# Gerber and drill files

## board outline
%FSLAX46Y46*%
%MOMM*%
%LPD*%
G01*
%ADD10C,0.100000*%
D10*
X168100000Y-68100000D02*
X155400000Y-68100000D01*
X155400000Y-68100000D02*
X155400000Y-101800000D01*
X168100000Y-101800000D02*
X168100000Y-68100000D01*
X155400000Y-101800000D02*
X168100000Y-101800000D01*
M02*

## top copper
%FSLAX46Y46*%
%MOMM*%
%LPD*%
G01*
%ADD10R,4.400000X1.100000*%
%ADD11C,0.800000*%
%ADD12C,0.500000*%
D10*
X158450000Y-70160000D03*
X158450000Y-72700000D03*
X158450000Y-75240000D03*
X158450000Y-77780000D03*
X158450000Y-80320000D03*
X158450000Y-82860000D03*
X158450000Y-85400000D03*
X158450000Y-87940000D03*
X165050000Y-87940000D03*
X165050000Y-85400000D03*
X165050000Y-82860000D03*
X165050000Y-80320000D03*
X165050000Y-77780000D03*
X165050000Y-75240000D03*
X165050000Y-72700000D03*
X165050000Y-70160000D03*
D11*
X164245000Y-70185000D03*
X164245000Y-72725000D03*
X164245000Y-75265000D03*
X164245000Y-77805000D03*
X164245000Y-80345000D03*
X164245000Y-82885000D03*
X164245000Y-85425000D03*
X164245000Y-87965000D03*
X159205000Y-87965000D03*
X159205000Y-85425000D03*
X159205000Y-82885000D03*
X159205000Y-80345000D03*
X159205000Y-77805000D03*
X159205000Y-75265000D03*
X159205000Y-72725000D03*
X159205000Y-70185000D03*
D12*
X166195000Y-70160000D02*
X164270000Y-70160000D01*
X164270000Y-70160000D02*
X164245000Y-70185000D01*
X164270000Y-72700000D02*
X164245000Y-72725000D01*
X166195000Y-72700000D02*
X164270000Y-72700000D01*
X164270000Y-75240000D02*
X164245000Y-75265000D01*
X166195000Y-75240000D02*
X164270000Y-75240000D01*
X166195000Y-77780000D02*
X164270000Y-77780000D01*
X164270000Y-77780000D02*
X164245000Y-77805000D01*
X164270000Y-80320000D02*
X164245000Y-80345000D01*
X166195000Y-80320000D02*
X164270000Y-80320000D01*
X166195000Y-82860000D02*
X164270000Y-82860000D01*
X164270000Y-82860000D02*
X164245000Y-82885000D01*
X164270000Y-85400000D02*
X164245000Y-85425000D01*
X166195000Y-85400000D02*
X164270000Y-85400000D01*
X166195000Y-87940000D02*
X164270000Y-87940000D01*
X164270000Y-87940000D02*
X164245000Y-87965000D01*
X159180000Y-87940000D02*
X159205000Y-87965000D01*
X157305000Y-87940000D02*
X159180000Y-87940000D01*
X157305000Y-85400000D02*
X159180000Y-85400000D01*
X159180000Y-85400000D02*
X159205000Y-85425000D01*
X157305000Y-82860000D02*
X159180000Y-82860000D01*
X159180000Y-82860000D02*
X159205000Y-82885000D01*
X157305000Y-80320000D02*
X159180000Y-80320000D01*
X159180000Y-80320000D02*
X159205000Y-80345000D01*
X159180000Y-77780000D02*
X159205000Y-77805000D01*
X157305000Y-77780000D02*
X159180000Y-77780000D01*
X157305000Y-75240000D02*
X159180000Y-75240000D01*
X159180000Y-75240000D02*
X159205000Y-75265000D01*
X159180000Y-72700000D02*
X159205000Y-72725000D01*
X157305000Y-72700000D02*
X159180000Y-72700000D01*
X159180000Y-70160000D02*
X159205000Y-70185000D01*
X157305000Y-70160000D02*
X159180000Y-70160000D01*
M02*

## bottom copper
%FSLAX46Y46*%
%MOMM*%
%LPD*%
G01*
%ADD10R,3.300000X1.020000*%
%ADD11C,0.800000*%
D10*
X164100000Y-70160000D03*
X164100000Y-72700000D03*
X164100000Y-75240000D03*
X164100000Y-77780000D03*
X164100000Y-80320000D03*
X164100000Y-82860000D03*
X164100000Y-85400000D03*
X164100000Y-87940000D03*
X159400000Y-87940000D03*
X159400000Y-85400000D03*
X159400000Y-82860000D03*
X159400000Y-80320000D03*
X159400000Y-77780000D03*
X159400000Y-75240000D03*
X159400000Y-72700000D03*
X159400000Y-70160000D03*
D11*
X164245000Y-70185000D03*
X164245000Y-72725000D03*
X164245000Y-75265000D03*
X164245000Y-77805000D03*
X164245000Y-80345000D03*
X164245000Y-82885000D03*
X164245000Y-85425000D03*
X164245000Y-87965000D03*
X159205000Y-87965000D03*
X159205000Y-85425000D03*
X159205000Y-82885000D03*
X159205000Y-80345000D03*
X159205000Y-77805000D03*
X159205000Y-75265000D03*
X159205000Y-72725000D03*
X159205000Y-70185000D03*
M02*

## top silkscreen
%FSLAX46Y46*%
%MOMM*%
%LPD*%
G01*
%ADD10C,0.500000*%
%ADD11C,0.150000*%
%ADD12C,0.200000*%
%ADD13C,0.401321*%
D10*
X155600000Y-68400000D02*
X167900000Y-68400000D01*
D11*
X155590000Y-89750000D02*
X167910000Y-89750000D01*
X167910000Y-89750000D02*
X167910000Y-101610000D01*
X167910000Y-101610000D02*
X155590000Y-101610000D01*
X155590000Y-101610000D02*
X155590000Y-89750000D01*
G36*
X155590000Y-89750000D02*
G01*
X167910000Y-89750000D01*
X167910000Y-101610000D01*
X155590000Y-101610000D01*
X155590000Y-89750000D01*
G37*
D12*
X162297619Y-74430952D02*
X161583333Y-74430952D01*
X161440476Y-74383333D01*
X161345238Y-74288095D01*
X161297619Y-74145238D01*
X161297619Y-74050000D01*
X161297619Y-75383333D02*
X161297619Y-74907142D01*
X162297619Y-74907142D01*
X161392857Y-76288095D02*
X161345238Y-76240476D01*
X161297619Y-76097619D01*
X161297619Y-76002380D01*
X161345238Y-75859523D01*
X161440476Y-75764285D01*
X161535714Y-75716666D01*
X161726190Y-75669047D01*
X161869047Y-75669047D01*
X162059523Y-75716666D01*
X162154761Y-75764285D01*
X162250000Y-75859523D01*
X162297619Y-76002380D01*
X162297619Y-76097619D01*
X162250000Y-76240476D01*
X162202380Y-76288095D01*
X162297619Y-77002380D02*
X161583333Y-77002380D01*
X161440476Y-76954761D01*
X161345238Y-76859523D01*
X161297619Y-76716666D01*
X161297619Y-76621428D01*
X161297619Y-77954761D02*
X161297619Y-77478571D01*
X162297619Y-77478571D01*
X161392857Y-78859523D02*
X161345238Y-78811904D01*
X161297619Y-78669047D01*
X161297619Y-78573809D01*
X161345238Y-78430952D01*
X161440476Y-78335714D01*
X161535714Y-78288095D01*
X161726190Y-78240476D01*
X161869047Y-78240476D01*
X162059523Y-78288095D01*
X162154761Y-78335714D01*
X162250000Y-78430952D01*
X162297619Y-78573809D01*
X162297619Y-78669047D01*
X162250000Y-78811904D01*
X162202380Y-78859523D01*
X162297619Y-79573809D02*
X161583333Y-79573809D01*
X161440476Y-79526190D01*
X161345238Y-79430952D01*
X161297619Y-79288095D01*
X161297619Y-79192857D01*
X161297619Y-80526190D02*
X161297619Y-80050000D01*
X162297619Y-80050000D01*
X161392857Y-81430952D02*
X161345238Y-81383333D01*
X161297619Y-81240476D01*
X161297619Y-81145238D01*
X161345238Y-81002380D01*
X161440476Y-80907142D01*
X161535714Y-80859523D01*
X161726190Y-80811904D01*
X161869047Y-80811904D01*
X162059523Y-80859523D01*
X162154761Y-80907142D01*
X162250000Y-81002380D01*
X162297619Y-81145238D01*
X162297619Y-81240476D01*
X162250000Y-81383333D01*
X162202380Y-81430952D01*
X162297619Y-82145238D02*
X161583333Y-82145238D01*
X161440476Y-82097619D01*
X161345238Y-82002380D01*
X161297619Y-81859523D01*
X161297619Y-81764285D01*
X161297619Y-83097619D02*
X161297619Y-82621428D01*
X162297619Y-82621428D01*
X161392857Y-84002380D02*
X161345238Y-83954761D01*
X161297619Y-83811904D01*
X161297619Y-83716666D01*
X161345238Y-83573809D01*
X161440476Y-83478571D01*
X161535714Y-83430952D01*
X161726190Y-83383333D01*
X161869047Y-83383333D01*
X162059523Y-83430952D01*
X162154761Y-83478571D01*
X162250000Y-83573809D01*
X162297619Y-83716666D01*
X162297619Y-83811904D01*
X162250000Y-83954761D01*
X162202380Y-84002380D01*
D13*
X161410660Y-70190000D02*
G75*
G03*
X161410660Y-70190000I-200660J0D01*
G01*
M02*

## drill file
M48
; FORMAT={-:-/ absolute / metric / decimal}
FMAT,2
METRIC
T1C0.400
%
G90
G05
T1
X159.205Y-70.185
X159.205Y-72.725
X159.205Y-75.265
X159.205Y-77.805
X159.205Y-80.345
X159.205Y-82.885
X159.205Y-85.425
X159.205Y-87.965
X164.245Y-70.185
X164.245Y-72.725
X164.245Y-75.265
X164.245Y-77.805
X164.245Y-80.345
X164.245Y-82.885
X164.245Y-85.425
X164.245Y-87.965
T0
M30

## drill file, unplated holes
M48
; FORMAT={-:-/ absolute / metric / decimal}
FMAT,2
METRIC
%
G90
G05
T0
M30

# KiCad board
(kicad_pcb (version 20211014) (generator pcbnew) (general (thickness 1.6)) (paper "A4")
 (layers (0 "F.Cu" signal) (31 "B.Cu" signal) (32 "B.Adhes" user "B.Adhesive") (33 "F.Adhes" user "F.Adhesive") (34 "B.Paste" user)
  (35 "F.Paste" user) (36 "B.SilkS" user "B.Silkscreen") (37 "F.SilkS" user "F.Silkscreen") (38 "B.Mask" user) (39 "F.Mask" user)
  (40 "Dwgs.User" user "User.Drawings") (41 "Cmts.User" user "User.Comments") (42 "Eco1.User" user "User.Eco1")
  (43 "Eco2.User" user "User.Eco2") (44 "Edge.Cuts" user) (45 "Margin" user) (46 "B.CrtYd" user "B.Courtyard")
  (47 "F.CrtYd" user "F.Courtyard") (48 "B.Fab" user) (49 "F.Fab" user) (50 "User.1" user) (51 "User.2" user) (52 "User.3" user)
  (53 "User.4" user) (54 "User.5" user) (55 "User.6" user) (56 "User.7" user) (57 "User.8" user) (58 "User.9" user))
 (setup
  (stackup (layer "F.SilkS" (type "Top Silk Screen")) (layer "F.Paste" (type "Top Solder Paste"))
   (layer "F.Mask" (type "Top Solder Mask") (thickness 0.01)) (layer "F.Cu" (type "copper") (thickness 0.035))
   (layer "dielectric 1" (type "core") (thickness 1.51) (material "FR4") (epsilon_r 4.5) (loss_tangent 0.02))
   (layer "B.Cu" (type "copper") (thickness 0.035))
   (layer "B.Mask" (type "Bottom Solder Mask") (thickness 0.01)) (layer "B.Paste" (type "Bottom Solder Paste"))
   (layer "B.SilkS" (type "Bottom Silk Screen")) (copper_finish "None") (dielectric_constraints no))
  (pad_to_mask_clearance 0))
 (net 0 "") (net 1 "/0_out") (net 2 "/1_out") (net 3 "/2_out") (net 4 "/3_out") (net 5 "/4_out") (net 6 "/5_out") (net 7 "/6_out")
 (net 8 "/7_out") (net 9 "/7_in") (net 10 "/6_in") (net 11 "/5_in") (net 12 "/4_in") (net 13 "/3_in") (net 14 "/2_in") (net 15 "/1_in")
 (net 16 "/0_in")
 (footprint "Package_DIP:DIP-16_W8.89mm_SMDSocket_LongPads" (layer "F.Cu") (at 161.75 79.05)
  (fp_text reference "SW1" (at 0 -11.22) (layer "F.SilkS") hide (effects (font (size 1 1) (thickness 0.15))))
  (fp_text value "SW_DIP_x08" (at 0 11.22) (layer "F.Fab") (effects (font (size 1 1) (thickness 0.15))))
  (fp_circle (center -0.54 -8.86) (end -0.198679 -8.86) (layer "F.SilkS") (width 0.12) (fill solid))
  (pad "1" smd rect (at -3.3 -8.89) (size 4.4 1.1) (layers "F.Cu" "F.Paste" "F.Mask") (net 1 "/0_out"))
  (pad "2" smd rect (at -3.3 -6.35) (size 4.4 1.1) (layers "F.Cu" "F.Paste" "F.Mask") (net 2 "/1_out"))
  (pad "3" smd rect (at -3.3 -3.81) (size 4.4 1.1) (layers "F.Cu" "F.Paste" "F.Mask") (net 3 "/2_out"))
  (pad "4" smd rect (at -3.3 -1.27) (size 4.4 1.1) (layers "F.Cu" "F.Paste" "F.Mask") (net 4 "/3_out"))
  (pad "5" smd rect (at -3.3 1.27) (size 4.4 1.1) (layers "F.Cu" "F.Paste" "F.Mask") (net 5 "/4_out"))
  (pad "6" smd rect (at -3.3 3.81) (size 4.4 1.1) (layers "F.Cu" "F.Paste" "F.Mask") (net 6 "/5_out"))
  (pad "7" smd rect (at -3.3 6.35) (size 4.4 1.1) (layers "F.Cu" "F.Paste" "F.Mask") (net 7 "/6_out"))
  (pad "8" smd rect (at -3.3 8.89) (size 4.4 1.1) (layers "F.Cu" "F.Paste" "F.Mask") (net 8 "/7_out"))
  (pad "9" smd rect (at 3.3 8.89) (size 4.4 1.1) (layers "F.Cu" "F.Paste" "F.Mask") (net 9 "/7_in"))
  (pad "10" smd rect (at 3.3 6.35) (size 4.4 1.1) (layers "F.Cu" "F.Paste" "F.Mask") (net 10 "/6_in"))
  (pad "11" smd rect (at 3.3 3.81) (size 4.4 1.1) (layers "F.Cu" "F.Paste" "F.Mask") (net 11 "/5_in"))
  (pad "12" smd rect (at 3.3 1.27) (size 4.4 1.1) (layers "F.Cu" "F.Paste" "F.Mask") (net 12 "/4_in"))
  (pad "13" smd rect (at 3.3 -1.27) (size 4.4 1.1) (layers "F.Cu" "F.Paste" "F.Mask") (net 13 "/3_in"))
  (pad "14" smd rect (at 3.3 -3.81) (size 4.4 1.1) (layers "F.Cu" "F.Paste" "F.Mask") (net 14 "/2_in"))
  (pad "15" smd rect (at 3.3 -6.35) (size 4.4 1.1) (layers "F.Cu" "F.Paste" "F.Mask") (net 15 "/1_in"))
  (pad "16" smd rect (at 3.3 -8.89) (size 4.4 1.1) (layers "F.Cu" "F.Paste" "F.Mask") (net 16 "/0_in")))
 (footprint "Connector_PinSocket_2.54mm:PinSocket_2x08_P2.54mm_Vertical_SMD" (layer "B.Cu") (at 161.725 79.075 180)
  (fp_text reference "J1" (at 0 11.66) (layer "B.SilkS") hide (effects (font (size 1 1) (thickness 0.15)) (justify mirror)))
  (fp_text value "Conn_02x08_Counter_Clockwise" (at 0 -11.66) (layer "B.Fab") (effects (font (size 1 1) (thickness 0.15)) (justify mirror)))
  (pad "1" smd rect (at -2.375 8.915 180) (size 3.3 1.02) (layers "B.Cu" "B.Paste" "B.Mask") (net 16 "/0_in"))
  (pad "2" smd rect (at -2.375 6.375 180) (size 3.3 1.02) (layers "B.Cu" "B.Paste" "B.Mask") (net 15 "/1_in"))
  (pad "3" smd rect (at -2.375 3.835 180) (size 3.3 1.02) (layers "B.Cu" "B.Paste" "B.Mask") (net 14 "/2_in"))
  (pad "4" smd rect (at -2.375 1.295 180) (size 3.3 1.02) (layers "B.Cu" "B.Paste" "B.Mask") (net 13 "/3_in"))
  (pad "5" smd rect (at -2.375 -1.245 180) (size 3.3 1.02) (layers "B.Cu" "B.Paste" "B.Mask") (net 12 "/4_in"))
  (pad "6" smd rect (at -2.375 -3.785 180) (size 3.3 1.02) (layers "B.Cu" "B.Paste" "B.Mask") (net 11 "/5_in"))
  (pad "7" smd rect (at -2.375 -6.325 180) (size 3.3 1.02) (layers "B.Cu" "B.Paste" "B.Mask") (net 10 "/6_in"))
  (pad "8" smd rect (at -2.375 -8.865 180) (size 3.3 1.02) (layers "B.Cu" "B.Paste" "B.Mask") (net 9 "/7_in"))
  (pad "9" smd rect (at 2.325 -8.865 180) (size 3.3 1.02) (layers "B.Cu" "B.Paste" "B.Mask") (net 8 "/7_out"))
  (pad "10" smd rect (at 2.325 -6.325 180) (size 3.3 1.02) (layers "B.Cu" "B.Paste" "B.Mask") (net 7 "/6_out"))
  (pad "11" smd rect (at 2.325 -3.785 180) (size 3.3 1.02) (layers "B.Cu" "B.Paste" "B.Mask") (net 6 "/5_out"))
  (pad "12" smd rect (at 2.325 -1.245 180) (size 3.3 1.02) (layers "B.Cu" "B.Paste" "B.Mask") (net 5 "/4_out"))
  (pad "13" smd rect (at 2.325 1.295 180) (size 3.3 1.02) (layers "B.Cu" "B.Paste" "B.Mask") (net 4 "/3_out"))
  (pad "14" smd rect (at 2.325 3.835 180) (size 3.3 1.02) (layers "B.Cu" "B.Paste" "B.Mask") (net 3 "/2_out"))
  (pad "15" smd rect (at 2.325 6.375 180) (size 3.3 1.02) (layers "B.Cu" "B.Paste" "B.Mask") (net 2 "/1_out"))
  (pad "16" smd rect (at 2.325 8.915 180) (size 3.3 1.02) (layers "B.Cu" "B.Paste" "B.Mask") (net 1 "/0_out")))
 (gr_line (start 155.6 68.4) (end 167.9 68.4) (layer "F.SilkS") (width 0.5))
 (gr_rect (start 155.59 89.75) (end 167.91 101.61) (layer "F.SilkS") (width 0.15) (fill solid))
 (gr_line (start 168.1 68.1) (end 155.4 68.1) (layer "Edge.Cuts") (width 0.1))
 (gr_line (start 155.4 68.1) (end 155.4 101.8) (layer "Edge.Cuts") (width 0.1))
 (gr_line (start 168.1 101.8) (end 168.1 68.1) (layer "Edge.Cuts") (width 0.1))
 (gr_line (start 155.4 101.8) (end 168.1 101.8) (layer "Edge.Cuts") (width 0.1))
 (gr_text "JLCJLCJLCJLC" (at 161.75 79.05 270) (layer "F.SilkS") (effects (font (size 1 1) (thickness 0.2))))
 (segment (start 166.195 70.16) (end 164.27 70.16) (width 0.5) (layer "F.Cu") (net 16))
 (segment (start 164.27 70.16) (end 164.245 70.185) (width 0.5) (layer "F.Cu") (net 16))
 (via (at 164.245 70.185) (size 0.8) (drill 0.4) (layers "F.Cu" "B.Cu") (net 16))
 (segment (start 164.27 72.7) (end 164.245 72.725) (width 0.5) (layer "F.Cu") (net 15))
 (segment (start 166.195 72.7) (end 164.27 72.7) (width 0.5) (layer "F.Cu") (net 15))
 (via (at 164.245 72.725) (size 0.8) (drill 0.4) (layers "F.Cu" "B.Cu") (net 15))
 (segment (start 164.27 75.24) (end 164.245 75.265) (width 0.5) (layer "F.Cu") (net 14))
 (segment (start 166.195 75.24) (end 164.27 75.24) (width 0.5) (layer "F.Cu") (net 14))
 (via (at 164.245 75.265) (size 0.8) (drill 0.4) (layers "F.Cu" "B.Cu") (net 14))
 (segment (start 166.195 77.78) (end 164.27 77.78) (width 0.5) (layer "F.Cu") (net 13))
 (segment (start 164.27 77.78) (end 164.245 77.805) (width 0.5) (layer "F.Cu") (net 13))
 (via (at 164.245 77.805) (size 0.8) (drill 0.4) (layers "F.Cu" "B.Cu") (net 13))
 (segment (start 164.27 80.32) (end 164.245 80.345) (width 0.5) (layer "F.Cu") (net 12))
 (segment (start 166.195 80.32) (end 164.27 80.32) (width 0.5) (layer "F.Cu") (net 12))
 (via (at 164.245 80.345) (size 0.8) (drill 0.4) (layers "F.Cu" "B.Cu") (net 12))
 (segment (start 166.195 82.86) (end 164.27 82.86) (width 0.5) (layer "F.Cu") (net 11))
 (segment (start 164.27 82.86) (end 164.245 82.885) (width 0.5) (layer "F.Cu") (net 11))
 (via (at 164.245 82.885) (size 0.8) (drill 0.4) (layers "F.Cu" "B.Cu") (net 11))
 (segment (start 164.27 85.4) (end 164.245 85.425) (width 0.5) (layer "F.Cu") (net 10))
 (segment (start 166.195 85.4) (end 164.27 85.4) (width 0.5) (layer "F.Cu") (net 10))
 (via (at 164.245 85.425) (size 0.8) (drill 0.4) (layers "F.Cu" "B.Cu") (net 10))
 (segment (start 166.195 87.94) (end 164.27 87.94) (width 0.5) (layer "F.Cu") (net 9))
 (segment (start 164.27 87.94) (end 164.245 87.965) (width 0.5) (layer "F.Cu") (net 9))
 (via (at 164.245 87.965) (size 0.8) (drill 0.4) (layers "F.Cu" "B.Cu") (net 9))
 (segment (start 159.18 87.94) (end 159.205 87.965) (width 0.5) (layer "F.Cu") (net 8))
 (segment (start 157.305 87.94) (end 159.18 87.94) (width 0.5) (layer "F.Cu") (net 8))
 (via (at 159.205 87.965) (size 0.8) (drill 0.4) (layers "F.Cu" "B.Cu") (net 8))
 (segment (start 157.305 85.4) (end 159.18 85.4) (width 0.5) (layer "F.Cu") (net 7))
 (segment (start 159.18 85.4) (end 159.205 85.425) (width 0.5) (layer "F.Cu") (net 7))
 (via (at 159.205 85.425) (size 0.8) (drill 0.4) (layers "F.Cu" "B.Cu") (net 7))
 (segment (start 157.305 82.86) (end 159.18 82.86) (width 0.5) (layer "F.Cu") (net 6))
 (segment (start 159.18 82.86) (end 159.205 82.885) (width 0.5) (layer "F.Cu") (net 6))
 (via (at 159.205 82.885) (size 0.8) (drill 0.4) (layers "F.Cu" "B.Cu") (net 6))
 (segment (start 157.305 80.32) (end 159.18 80.32) (width 0.5) (layer "F.Cu") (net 5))
 (segment (start 159.18 80.32) (end 159.205 80.345) (width 0.5) (layer "F.Cu") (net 5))
 (via (at 159.205 80.345) (size 0.8) (drill 0.4) (layers "F.Cu" "B.Cu") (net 5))
 (segment (start 159.18 77.78) (end 159.205 77.805) (width 0.5) (layer "F.Cu") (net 4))
 (segment (start 157.305 77.78) (end 159.18 77.78) (width 0.5) (layer "F.Cu") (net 4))
 (via (at 159.205 77.805) (size 0.8) (drill 0.4) (layers "F.Cu" "B.Cu") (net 4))
 (segment (start 157.305 75.24) (end 159.18 75.24) (width 0.5) (layer "F.Cu") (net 3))
 (segment (start 159.18 75.24) (end 159.205 75.265) (width 0.5) (layer "F.Cu") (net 3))
 (via (at 159.205 75.265) (size 0.8) (drill 0.4) (layers "F.Cu" "B.Cu") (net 3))
 (segment (start 159.18 72.7) (end 159.205 72.725) (width 0.5) (layer "F.Cu") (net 2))
 (segment (start 157.305 72.7) (end 159.18 72.7) (width 0.5) (layer "F.Cu") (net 2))
 (via (at 159.205 72.725) (size 0.8) (drill 0.4) (layers "F.Cu" "B.Cu") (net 2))
 (segment (start 159.18 70.16) (end 159.205 70.185) (width 0.5) (layer "F.Cu") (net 1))
 (segment (start 157.305 70.16) (end 159.18 70.16) (width 0.5) (layer "F.Cu") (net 1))
 (via (at 159.205 70.185) (size 0.8) (drill 0.4) (layers "F.Cu" "B.Cu") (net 1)))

